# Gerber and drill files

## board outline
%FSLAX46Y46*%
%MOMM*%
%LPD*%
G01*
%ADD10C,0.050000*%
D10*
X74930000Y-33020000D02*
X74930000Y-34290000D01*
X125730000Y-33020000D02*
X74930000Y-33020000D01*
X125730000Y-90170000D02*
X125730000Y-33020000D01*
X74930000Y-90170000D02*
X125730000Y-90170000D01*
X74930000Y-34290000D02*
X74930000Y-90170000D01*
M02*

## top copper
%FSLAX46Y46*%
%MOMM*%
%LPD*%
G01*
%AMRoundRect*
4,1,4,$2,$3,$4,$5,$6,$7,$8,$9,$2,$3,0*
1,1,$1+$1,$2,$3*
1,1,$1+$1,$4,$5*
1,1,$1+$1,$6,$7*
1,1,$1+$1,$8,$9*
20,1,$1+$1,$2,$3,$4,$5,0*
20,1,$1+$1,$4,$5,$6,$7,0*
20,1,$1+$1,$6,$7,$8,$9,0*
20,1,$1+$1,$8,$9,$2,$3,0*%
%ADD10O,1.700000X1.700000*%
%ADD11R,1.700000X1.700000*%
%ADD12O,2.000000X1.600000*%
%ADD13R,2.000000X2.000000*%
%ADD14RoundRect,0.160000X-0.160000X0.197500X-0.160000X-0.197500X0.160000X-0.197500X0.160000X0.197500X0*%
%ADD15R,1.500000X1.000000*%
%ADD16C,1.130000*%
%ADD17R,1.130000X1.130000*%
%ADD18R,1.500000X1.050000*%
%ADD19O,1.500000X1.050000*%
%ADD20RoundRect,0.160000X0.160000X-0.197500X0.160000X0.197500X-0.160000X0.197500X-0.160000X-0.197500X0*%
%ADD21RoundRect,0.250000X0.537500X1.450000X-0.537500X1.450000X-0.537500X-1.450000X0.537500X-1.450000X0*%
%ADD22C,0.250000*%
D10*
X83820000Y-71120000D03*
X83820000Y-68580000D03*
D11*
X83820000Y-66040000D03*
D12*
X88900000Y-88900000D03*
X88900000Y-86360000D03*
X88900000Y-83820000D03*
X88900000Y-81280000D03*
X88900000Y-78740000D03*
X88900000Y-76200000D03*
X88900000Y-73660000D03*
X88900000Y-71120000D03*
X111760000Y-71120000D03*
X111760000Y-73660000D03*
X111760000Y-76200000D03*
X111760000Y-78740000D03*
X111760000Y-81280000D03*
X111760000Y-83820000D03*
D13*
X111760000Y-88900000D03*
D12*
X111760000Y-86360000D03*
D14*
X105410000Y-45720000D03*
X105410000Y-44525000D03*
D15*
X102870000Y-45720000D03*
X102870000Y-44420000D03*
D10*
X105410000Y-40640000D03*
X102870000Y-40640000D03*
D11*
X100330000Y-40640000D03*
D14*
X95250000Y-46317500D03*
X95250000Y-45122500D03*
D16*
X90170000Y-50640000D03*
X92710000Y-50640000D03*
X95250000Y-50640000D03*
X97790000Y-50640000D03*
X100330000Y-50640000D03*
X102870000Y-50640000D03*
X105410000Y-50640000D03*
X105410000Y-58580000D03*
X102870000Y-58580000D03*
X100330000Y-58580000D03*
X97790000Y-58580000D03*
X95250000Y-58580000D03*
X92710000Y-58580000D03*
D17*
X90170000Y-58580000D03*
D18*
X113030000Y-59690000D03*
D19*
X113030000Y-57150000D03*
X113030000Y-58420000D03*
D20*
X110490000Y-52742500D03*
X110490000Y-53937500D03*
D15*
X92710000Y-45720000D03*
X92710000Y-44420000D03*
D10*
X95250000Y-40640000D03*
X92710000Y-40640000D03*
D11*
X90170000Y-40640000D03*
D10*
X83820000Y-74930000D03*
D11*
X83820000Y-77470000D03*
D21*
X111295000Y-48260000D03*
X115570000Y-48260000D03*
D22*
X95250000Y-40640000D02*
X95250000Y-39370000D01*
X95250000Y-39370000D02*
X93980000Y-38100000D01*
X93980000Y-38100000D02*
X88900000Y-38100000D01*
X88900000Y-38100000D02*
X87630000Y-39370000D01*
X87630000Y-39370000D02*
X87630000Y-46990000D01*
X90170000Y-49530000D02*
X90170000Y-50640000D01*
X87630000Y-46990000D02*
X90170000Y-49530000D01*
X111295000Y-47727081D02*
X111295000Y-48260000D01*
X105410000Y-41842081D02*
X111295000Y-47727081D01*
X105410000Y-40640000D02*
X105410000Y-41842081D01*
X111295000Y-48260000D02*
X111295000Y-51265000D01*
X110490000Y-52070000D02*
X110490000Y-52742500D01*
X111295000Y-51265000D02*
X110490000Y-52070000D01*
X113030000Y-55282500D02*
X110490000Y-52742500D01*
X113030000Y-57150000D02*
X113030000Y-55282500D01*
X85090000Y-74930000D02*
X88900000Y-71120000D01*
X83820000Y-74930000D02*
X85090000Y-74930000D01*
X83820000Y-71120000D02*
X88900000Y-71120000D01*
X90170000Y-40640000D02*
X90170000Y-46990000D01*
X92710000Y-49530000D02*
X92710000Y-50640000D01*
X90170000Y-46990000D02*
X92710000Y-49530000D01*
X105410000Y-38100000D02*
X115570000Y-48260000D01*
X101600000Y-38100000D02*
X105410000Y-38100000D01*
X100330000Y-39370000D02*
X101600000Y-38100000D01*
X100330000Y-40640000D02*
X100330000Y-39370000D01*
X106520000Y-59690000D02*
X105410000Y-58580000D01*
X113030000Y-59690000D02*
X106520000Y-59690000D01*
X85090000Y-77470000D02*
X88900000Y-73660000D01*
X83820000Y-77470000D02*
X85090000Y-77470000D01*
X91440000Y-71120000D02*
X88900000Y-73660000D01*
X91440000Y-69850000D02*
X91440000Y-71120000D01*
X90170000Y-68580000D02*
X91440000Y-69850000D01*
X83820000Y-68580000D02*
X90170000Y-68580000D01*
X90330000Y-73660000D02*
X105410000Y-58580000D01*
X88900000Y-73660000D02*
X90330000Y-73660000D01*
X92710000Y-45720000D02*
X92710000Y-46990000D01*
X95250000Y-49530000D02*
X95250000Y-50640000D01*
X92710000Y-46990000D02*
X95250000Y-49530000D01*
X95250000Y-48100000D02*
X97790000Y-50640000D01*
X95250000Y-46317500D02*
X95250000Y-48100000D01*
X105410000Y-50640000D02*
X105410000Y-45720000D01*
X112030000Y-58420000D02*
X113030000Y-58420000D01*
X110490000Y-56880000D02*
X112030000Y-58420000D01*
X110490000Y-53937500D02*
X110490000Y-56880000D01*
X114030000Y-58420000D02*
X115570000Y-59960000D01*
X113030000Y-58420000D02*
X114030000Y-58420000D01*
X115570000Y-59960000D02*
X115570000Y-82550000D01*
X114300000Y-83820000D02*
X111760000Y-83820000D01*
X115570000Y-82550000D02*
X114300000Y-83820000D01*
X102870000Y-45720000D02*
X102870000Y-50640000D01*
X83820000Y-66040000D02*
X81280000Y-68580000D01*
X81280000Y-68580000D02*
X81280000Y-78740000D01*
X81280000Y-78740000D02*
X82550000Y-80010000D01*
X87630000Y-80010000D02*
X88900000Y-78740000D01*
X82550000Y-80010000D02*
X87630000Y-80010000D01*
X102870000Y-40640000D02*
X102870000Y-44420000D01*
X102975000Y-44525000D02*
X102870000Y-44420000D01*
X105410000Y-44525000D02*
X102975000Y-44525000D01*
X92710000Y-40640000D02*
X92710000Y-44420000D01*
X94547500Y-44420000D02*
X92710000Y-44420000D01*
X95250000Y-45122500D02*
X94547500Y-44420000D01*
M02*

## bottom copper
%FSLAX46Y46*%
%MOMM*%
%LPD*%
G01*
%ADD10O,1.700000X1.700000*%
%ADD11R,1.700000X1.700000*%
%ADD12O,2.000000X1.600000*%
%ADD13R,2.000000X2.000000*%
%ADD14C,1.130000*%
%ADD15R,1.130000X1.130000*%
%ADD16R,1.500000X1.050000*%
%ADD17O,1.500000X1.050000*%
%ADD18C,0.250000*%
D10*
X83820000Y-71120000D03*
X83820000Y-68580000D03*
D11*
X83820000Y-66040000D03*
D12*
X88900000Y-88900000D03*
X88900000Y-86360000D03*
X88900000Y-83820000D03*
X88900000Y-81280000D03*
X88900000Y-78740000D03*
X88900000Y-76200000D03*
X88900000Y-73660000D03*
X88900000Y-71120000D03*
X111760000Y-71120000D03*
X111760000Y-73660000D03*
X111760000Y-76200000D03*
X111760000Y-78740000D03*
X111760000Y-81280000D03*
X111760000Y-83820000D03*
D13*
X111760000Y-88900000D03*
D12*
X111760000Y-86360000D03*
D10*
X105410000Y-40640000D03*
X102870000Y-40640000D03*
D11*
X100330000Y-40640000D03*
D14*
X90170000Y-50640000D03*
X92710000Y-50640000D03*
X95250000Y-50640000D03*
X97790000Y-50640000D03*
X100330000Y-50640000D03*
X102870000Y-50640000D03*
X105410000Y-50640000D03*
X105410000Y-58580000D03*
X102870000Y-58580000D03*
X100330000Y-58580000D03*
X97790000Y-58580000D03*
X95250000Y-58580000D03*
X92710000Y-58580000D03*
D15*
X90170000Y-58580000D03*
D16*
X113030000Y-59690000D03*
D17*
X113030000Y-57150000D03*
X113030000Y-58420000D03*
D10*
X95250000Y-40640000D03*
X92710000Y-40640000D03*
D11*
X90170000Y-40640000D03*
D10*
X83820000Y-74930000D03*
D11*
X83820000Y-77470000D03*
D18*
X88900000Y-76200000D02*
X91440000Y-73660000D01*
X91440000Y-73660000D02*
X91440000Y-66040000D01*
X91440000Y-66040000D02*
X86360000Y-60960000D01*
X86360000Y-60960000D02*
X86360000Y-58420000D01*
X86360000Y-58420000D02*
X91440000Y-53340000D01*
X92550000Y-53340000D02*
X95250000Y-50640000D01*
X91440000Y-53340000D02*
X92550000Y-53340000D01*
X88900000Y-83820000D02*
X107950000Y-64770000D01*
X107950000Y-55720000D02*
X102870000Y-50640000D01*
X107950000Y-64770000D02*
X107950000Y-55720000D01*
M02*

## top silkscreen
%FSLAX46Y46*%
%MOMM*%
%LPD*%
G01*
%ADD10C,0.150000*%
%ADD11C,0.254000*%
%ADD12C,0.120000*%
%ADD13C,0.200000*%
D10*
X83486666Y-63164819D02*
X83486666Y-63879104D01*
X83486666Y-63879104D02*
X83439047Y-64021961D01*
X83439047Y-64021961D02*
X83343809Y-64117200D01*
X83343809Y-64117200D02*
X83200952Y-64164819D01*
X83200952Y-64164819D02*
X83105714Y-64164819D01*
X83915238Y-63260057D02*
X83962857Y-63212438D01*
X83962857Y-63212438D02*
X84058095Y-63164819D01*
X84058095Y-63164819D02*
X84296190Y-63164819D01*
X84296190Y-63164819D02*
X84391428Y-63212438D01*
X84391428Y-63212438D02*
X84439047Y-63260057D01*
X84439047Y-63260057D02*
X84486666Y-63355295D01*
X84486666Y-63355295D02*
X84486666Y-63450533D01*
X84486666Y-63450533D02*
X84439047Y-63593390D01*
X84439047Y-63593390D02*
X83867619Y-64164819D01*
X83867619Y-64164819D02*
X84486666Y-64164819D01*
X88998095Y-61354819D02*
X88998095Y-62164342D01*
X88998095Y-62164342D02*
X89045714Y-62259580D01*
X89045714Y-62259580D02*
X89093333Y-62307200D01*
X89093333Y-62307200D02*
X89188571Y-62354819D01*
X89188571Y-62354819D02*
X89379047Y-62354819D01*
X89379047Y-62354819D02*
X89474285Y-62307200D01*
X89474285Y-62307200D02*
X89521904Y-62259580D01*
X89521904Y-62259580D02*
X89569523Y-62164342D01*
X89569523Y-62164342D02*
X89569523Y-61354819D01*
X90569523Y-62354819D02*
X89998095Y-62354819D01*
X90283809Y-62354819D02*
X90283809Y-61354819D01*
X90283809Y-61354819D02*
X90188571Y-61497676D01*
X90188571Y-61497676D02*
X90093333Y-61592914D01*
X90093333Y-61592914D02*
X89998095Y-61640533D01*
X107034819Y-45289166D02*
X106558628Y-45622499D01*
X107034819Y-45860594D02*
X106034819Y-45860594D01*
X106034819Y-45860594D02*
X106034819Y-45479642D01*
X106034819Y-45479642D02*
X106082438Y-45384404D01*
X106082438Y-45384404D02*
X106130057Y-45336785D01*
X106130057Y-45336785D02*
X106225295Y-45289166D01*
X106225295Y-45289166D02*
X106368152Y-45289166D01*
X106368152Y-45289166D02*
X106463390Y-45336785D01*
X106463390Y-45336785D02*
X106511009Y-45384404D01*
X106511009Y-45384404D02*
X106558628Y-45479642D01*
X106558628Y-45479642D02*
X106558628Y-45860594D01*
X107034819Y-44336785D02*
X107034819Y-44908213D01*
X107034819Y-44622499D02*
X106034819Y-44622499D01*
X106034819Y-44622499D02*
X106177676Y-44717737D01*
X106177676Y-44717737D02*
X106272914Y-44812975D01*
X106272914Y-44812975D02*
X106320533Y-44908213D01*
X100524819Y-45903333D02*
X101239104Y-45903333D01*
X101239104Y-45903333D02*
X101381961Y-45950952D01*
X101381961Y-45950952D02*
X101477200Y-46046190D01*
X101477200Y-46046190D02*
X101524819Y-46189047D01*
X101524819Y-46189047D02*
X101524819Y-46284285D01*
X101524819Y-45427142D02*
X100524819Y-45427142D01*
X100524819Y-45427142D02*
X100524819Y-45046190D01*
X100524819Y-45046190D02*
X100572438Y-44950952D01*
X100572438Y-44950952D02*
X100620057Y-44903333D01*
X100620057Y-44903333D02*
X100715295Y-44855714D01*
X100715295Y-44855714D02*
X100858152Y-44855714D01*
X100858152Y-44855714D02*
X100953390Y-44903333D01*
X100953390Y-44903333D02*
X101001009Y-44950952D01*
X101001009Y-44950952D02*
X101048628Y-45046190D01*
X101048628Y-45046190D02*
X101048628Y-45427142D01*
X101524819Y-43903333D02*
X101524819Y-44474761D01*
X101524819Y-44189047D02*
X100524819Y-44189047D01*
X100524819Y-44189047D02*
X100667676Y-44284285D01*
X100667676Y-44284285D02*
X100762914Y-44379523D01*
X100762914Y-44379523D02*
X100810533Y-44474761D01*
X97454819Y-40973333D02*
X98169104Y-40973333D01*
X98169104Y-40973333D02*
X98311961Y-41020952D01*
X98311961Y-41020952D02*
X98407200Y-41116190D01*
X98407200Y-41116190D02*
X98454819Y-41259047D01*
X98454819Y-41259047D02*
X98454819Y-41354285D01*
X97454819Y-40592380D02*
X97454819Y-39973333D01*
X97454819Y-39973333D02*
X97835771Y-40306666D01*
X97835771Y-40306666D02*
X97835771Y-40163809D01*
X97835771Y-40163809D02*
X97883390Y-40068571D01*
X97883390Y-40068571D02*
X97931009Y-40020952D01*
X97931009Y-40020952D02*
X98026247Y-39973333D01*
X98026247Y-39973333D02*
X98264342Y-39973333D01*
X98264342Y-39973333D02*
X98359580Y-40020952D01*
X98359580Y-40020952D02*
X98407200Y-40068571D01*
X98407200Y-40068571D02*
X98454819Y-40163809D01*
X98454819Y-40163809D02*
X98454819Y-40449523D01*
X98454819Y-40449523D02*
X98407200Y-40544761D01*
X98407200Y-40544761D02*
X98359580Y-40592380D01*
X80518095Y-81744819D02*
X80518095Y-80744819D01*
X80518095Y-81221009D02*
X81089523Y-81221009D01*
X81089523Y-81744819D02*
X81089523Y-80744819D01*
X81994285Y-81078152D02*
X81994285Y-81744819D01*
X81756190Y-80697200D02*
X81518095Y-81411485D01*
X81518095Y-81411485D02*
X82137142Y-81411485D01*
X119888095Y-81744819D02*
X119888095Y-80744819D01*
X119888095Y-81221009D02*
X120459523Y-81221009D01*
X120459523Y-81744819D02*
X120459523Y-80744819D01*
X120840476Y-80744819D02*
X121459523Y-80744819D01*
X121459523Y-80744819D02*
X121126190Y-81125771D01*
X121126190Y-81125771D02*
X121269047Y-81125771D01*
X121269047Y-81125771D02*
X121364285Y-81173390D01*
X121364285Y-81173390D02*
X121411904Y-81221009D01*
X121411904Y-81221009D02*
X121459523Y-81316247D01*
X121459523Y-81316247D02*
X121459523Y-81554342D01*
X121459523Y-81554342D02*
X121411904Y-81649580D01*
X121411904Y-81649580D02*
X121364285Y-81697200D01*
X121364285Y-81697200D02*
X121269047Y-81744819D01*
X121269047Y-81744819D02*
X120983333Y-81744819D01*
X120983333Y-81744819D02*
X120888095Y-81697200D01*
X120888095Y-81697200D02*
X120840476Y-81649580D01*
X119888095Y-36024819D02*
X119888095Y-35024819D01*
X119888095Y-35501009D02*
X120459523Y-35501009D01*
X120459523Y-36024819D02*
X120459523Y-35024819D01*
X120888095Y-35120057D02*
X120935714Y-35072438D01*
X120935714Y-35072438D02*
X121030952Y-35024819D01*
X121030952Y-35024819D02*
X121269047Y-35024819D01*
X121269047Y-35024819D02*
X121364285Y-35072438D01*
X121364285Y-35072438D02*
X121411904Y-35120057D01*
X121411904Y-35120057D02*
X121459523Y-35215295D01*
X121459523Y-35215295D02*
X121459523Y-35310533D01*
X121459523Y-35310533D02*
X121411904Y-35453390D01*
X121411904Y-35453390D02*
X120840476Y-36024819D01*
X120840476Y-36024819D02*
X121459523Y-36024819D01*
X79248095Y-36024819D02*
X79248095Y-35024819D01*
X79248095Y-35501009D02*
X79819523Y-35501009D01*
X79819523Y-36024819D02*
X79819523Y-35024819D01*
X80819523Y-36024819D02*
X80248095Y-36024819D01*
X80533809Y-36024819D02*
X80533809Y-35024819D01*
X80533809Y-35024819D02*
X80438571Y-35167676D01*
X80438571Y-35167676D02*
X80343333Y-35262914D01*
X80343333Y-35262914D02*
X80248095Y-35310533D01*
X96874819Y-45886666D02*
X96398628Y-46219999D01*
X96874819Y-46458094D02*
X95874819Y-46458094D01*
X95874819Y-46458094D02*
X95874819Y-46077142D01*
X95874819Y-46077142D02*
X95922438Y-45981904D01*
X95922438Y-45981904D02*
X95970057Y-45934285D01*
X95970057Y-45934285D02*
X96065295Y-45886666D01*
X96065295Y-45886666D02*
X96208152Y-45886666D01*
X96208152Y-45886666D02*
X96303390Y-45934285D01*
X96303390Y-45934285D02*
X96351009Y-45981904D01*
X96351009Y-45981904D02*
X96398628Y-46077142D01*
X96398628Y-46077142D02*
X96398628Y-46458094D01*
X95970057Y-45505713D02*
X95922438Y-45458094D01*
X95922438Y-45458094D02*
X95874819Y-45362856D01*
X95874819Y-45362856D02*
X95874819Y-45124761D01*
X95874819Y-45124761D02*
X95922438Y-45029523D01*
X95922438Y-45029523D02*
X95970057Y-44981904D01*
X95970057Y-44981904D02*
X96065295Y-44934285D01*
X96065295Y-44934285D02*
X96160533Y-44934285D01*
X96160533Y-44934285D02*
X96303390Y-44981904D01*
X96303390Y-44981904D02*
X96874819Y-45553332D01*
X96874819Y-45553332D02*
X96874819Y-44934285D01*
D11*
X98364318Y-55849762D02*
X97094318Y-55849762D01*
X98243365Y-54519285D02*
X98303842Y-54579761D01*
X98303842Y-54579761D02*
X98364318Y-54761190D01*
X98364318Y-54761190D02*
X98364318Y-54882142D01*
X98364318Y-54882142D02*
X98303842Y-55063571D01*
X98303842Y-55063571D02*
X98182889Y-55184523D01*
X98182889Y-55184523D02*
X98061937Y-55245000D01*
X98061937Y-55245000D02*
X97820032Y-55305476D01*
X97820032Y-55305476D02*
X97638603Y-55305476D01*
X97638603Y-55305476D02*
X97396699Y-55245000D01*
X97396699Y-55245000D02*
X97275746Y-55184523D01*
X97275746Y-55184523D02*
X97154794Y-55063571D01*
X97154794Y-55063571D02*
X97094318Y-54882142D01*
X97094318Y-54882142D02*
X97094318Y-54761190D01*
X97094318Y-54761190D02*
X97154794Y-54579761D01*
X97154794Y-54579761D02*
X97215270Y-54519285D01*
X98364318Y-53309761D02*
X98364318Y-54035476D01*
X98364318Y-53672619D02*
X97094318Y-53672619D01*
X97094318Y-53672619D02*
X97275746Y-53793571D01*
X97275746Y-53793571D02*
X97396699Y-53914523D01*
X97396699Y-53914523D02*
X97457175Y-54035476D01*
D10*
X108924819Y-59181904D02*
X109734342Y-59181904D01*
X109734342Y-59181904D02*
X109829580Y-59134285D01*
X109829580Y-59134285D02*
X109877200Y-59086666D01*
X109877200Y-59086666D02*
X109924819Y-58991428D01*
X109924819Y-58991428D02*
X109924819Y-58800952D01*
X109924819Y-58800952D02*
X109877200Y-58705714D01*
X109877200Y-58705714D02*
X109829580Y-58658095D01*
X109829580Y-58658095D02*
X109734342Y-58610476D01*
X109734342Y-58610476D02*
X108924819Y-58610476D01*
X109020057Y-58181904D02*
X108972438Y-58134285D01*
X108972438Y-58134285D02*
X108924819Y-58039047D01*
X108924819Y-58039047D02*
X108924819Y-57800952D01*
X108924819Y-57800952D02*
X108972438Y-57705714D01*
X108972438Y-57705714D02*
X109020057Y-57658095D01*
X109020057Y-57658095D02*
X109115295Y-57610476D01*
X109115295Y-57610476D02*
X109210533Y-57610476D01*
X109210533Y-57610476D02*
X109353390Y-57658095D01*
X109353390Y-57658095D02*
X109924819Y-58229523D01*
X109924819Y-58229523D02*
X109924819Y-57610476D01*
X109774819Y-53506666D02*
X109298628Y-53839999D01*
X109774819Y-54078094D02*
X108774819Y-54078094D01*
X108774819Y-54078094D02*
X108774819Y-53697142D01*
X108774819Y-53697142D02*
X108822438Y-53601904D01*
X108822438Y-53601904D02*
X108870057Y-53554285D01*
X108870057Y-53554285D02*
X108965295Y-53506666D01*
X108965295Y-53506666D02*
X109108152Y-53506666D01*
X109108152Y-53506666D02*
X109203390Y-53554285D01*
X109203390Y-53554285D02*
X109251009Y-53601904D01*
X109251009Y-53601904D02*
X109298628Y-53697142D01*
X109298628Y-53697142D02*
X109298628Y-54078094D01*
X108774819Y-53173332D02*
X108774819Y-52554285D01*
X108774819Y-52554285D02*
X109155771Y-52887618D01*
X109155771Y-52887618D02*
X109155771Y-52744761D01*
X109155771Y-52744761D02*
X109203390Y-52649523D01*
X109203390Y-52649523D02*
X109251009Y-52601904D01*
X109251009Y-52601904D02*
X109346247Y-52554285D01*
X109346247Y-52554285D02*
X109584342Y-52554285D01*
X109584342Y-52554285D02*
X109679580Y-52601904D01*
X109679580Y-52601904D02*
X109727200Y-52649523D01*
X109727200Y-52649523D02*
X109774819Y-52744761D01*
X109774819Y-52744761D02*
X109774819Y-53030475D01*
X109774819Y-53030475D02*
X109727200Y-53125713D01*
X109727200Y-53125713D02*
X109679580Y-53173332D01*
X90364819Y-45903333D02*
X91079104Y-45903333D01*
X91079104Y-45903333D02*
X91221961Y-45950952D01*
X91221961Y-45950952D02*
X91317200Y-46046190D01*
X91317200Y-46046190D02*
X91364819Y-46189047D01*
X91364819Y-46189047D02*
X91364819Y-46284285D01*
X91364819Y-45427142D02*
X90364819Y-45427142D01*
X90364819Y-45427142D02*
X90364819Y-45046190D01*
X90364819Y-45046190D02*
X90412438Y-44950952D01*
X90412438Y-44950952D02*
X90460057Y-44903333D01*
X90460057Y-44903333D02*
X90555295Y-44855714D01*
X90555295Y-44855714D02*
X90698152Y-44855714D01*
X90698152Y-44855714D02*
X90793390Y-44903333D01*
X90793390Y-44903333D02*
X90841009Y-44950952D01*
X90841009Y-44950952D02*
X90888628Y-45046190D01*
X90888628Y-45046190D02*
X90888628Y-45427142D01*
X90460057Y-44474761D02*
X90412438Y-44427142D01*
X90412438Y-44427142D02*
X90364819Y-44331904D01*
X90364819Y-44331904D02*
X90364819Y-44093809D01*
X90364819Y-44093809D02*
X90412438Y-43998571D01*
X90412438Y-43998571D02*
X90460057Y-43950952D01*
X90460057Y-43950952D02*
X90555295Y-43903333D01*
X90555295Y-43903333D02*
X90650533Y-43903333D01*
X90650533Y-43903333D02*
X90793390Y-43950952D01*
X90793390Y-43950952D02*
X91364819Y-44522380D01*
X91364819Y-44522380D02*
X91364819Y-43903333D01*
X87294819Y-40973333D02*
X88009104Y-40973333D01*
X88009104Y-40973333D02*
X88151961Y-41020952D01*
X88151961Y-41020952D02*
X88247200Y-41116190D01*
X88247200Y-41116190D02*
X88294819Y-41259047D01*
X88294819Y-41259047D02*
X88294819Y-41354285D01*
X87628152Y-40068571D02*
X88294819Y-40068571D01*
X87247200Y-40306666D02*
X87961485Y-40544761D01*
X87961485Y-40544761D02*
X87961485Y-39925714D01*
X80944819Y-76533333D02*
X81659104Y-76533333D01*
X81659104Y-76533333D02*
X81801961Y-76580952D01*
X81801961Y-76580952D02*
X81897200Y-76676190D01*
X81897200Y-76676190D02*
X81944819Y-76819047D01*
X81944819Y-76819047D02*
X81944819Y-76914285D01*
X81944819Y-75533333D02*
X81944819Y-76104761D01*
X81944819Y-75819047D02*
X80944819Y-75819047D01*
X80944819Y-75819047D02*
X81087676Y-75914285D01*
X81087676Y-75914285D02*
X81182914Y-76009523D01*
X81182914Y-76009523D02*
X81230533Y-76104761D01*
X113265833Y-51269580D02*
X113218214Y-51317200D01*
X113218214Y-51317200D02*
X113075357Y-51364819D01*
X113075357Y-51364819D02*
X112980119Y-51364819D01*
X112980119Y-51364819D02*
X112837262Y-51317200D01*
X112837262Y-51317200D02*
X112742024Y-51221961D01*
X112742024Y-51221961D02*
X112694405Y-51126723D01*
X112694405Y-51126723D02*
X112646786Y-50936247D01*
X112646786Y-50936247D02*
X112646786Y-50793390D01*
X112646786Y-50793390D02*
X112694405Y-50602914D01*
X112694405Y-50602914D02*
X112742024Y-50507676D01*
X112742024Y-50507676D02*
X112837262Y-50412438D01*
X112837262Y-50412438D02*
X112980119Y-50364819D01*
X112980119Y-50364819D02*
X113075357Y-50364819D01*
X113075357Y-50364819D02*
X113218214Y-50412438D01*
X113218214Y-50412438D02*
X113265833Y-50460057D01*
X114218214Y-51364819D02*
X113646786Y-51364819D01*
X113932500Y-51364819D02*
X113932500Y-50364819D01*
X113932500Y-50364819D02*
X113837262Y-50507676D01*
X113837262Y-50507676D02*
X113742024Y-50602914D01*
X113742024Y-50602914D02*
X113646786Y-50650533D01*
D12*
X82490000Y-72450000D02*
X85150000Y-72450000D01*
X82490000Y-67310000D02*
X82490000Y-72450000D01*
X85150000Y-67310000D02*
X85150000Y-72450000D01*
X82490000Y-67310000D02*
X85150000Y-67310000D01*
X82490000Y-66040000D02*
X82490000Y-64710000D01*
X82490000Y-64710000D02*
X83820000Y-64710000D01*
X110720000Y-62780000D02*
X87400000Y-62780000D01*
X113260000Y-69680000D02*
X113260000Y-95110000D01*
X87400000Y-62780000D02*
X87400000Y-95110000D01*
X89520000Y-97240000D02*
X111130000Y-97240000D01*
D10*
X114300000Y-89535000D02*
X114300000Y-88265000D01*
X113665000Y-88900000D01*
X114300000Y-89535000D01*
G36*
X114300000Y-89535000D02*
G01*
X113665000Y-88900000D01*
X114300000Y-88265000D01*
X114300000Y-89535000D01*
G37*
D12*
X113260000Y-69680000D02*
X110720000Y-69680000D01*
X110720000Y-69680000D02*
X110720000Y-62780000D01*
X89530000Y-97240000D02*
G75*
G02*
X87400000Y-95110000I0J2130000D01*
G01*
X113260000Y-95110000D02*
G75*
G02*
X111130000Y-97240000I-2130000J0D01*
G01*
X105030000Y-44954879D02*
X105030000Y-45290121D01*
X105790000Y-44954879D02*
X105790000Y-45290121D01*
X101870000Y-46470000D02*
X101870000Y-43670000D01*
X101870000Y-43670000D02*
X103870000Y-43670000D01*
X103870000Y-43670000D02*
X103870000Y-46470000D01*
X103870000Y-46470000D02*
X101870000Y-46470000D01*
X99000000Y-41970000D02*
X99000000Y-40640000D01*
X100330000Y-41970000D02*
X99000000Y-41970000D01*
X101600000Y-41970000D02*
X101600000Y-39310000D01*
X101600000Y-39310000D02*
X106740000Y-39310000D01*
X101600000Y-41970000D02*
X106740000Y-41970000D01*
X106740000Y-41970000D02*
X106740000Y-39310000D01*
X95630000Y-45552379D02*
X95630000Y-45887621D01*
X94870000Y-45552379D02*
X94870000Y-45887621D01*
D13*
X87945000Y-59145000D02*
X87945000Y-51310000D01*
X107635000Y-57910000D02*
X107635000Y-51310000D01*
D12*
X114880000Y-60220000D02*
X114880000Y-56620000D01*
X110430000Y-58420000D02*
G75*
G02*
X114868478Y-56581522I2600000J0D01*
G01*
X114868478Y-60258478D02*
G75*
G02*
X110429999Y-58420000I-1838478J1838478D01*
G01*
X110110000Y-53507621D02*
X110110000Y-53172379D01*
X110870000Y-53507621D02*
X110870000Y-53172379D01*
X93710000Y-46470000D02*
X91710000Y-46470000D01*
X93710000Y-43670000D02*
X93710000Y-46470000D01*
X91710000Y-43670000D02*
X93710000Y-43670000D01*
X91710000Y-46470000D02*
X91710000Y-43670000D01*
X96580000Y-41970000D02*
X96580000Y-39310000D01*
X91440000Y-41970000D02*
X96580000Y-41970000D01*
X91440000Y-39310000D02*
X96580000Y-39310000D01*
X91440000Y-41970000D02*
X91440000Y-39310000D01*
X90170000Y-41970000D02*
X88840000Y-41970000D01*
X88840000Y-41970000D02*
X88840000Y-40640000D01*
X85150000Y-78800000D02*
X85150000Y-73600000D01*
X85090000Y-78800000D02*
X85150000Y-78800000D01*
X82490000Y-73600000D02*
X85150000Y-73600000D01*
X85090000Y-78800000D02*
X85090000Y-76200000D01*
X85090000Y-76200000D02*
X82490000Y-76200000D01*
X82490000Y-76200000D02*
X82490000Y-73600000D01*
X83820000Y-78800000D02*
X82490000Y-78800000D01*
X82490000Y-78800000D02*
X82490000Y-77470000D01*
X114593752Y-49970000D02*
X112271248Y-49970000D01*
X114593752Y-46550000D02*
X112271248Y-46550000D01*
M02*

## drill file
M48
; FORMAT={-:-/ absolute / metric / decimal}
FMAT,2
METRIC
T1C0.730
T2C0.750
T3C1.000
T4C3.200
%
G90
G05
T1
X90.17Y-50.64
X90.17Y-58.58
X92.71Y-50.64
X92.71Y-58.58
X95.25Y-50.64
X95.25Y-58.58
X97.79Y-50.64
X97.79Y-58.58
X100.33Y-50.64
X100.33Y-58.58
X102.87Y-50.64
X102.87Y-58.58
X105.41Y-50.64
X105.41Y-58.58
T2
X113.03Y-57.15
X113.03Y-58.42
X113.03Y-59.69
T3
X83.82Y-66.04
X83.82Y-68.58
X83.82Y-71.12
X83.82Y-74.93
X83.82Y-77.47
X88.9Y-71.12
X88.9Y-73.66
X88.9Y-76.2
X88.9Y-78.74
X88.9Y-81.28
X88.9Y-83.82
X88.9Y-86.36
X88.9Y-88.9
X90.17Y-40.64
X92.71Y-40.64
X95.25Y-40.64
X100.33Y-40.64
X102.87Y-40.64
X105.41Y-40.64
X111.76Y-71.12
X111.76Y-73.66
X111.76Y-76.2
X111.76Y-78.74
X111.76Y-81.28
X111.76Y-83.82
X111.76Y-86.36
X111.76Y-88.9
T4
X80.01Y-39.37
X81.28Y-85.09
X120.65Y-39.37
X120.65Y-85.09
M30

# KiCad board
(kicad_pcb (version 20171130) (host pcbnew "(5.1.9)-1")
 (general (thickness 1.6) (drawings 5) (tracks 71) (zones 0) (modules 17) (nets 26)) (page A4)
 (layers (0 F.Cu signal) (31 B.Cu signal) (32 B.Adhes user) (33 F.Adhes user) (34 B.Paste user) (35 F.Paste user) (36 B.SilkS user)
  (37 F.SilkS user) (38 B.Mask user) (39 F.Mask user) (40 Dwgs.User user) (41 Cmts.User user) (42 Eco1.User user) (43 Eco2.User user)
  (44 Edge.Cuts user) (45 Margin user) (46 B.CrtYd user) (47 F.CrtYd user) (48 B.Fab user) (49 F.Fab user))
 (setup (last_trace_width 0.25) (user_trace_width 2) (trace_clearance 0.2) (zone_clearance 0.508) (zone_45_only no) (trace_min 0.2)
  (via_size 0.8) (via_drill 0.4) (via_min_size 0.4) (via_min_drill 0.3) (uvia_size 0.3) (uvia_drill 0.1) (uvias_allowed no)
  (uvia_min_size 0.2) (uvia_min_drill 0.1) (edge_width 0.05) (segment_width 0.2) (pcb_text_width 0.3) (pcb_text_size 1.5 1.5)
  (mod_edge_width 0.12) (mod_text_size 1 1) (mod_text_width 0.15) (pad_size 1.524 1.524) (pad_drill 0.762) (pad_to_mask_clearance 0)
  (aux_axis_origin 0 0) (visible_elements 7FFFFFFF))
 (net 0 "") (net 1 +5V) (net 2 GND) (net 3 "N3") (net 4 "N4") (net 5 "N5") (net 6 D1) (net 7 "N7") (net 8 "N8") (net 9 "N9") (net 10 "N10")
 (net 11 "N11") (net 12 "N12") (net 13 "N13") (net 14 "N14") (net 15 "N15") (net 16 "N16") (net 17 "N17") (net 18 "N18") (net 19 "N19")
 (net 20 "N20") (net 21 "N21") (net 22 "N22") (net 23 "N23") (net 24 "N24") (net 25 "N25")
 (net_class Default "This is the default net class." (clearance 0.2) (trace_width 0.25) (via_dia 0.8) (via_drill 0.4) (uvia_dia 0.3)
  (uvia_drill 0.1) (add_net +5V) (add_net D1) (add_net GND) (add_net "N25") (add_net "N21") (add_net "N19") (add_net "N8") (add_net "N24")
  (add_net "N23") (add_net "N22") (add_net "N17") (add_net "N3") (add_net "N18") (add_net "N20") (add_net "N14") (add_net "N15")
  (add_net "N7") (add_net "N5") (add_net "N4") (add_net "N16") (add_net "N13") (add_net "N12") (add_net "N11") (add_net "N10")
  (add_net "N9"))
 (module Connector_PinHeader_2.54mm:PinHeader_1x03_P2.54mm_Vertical (layer F.Cu) (at 83.82 66.04)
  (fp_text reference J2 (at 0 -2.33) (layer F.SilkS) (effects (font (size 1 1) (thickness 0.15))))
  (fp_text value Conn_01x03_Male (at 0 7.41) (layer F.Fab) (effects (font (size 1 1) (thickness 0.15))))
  (fp_line (start -1.33 6.41) (end 1.33 6.41) (layer F.SilkS) (width 0.12))
  (fp_line (start -1.33 1.27) (end -1.33 6.41) (layer F.SilkS) (width 0.12))
  (fp_line (start 1.33 1.27) (end 1.33 6.41) (layer F.SilkS) (width 0.12))
  (fp_line (start -1.33 1.27) (end 1.33 1.27) (layer F.SilkS) (width 0.12))
  (fp_line (start -1.33 0) (end -1.33 -1.33) (layer F.SilkS) (width 0.12))
  (fp_line (start -1.33 -1.33) (end 0 -1.33) (layer F.SilkS) (width 0.12))
  (pad 3 thru_hole oval (at 0 5.08) (size 1.7 1.7) (drill 1) (layers *.Cu *.Mask) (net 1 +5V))
  (pad 2 thru_hole oval (at 0 2.54) (size 1.7 1.7) (drill 1) (layers *.Cu *.Mask) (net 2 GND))
  (pad 1 thru_hole rect (at 0 0) (size 1.7 1.7) (drill 1) (layers *.Cu *.Mask) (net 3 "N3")))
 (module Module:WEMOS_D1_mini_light (layer F.Cu) (at 111.76 88.9 180)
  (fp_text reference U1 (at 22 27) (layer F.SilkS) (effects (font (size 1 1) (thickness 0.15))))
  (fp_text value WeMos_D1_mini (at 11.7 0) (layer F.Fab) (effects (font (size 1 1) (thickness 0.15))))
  (fp_line (start 1.04 26.12) (end 24.36 26.12) (layer F.SilkS) (width 0.12))
  (fp_line (start -1.5 19.22) (end -1.5 -6.21) (layer F.SilkS) (width 0.12))
  (fp_line (start 24.36 26.12) (end 24.36 -6.21) (layer F.SilkS) (width 0.12))
  (fp_line (start 22.24 -8.34) (end 0.63 -8.34) (layer F.SilkS) (width 0.12))
  (fp_poly (pts (xy -2.54 -0.635) (xy -2.54 0.635) (xy -1.905 0)) (layer F.SilkS) (width 0.15))
  (fp_line (start -1.5 19.22) (end 1.04 19.22) (layer F.SilkS) (width 0.12))
  (fp_line (start 1.04 19.22) (end 1.04 26.12) (layer F.SilkS) (width 0.12))
  (fp_arc (start 22.23 -6.21) (end 24.36 -6.21) (angle -90) (layer F.SilkS) (width 0.12))
  (fp_arc (start 0.63 -6.21) (end 0.63 -8.34) (angle -90) (layer F.SilkS) (width 0.12))
  (pad 16 thru_hole oval (at 22.86 0 180) (size 2 1.6) (drill 1) (layers *.Cu *.Mask) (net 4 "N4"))
  (pad 15 thru_hole oval (at 22.86 2.54 180) (size 2 1.6) (drill 1) (layers *.Cu *.Mask) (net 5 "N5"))
  (pad 14 thru_hole oval (at 22.86 5.08 180) (size 2 1.6) (drill 1) (layers *.Cu *.Mask) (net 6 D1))
  (pad 13 thru_hole oval (at 22.86 7.62 180) (size 2 1.6) (drill 1) (layers *.Cu *.Mask) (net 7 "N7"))
  (pad 12 thru_hole oval (at 22.86 10.16 180) (size 2 1.6) (drill 1) (layers *.Cu *.Mask) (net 3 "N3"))
  (pad 11 thru_hole oval (at 22.86 12.7 180) (size 2 1.6) (drill 1) (layers *.Cu *.Mask) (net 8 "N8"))
  (pad 10 thru_hole oval (at 22.86 15.24 180) (size 2 1.6) (drill 1) (layers *.Cu *.Mask) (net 2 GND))
  (pad 9 thru_hole oval (at 22.86 17.78 180) (size 2 1.6) (drill 1) (layers *.Cu *.Mask) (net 1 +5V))
  (pad 8 thru_hole oval (at 0 17.78 180) (size 2 1.6) (drill 1) (layers *.Cu *.Mask) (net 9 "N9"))
  (pad 7 thru_hole oval (at 0 15.24 180) (size 2 1.6) (drill 1) (layers *.Cu *.Mask) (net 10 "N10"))
  (pad 6 thru_hole oval (at 0 12.7 180) (size 2 1.6) (drill 1) (layers *.Cu *.Mask) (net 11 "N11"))
  (pad 5 thru_hole oval (at 0 10.16 180) (size 2 1.6) (drill 1) (layers *.Cu *.Mask) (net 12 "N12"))
  (pad 4 thru_hole oval (at 0 7.62 180) (size 2 1.6) (drill 1) (layers *.Cu *.Mask) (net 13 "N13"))
  (pad 3 thru_hole oval (at 0 5.08 180) (size 2 1.6) (drill 1) (layers *.Cu *.Mask) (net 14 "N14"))
  (pad 1 thru_hole rect (at 0 0 180) (size 2 2) (drill 1) (layers *.Cu *.Mask) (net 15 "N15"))
  (pad 2 thru_hole oval (at 0 2.54 180) (size 2 1.6) (drill 1) (layers *.Cu *.Mask) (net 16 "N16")))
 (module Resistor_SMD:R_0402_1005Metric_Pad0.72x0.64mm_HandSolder (layer F.Cu) (at 105.41 45.1225 270)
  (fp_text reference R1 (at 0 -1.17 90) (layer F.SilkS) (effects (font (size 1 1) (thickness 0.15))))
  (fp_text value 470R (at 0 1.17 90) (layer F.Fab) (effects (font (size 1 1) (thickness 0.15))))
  (fp_line (start -0.167621 0.38) (end 0.167621 0.38) (layer F.SilkS) (width 0.12))
  (fp_line (start -0.167621 -0.38) (end 0.167621 -0.38) (layer F.SilkS) (width 0.12))
  (pad 2 smd roundrect (at 0.5975 0 270) (size 0.715 0.64) (layers F.Cu F.Paste F.Mask) (roundrect_rratio 0.25) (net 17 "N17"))
  (pad 1 smd roundrect (at -0.5975 0 270) (size 0.715 0.64) (layers F.Cu F.Paste F.Mask) (roundrect_rratio 0.25) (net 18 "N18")))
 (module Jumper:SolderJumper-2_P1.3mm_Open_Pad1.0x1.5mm (layer F.Cu) (at 102.87 45.07 90)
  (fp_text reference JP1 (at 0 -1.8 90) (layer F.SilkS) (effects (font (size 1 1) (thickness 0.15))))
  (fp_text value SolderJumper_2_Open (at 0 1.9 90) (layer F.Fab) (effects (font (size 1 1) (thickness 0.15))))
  (fp_line (start -1.4 -1) (end 1.4 -1) (layer F.SilkS) (width 0.12))
  (fp_line (start 1.4 -1) (end 1.4 1) (layer F.SilkS) (width 0.12))
  (fp_line (start 1.4 1) (end -1.4 1) (layer F.SilkS) (width 0.12))
  (fp_line (start -1.4 1) (end -1.4 -1) (layer F.SilkS) (width 0.12))
  (pad 1 smd rect (at -0.65 0 90) (size 1 1.5) (layers F.Cu F.Mask) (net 6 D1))
  (pad 2 smd rect (at 0.65 0 90) (size 1 1.5) (layers F.Cu F.Mask) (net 18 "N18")))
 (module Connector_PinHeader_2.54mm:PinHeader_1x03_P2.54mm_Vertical (layer F.Cu) (at 100.33 40.64 90)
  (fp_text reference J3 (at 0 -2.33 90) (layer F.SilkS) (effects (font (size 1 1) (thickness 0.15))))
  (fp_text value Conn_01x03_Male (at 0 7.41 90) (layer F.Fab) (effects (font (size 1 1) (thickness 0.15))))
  (fp_line (start -1.33 -1.33) (end 0 -1.33) (layer F.SilkS) (width 0.12))
  (fp_line (start -1.33 0) (end -1.33 -1.33) (layer F.SilkS) (width 0.12))
  (fp_line (start -1.33 1.27) (end 1.33 1.27) (layer F.SilkS) (width 0.12))
  (fp_line (start 1.33 1.27) (end 1.33 6.41) (layer F.SilkS) (width 0.12))
  (fp_line (start -1.33 1.27) (end -1.33 6.41) (layer F.SilkS) (width 0.12))
  (fp_line (start -1.33 6.41) (end 1.33 6.41) (layer F.SilkS) (width 0.12))
  (pad 3 thru_hole oval (at 0 5.08 90) (size 1.7 1.7) (drill 1) (layers *.Cu *.Mask) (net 1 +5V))
  (pad 2 thru_hole oval (at 0 2.54 90) (size 1.7 1.7) (drill 1) (layers *.Cu *.Mask) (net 18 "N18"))
  (pad 1 thru_hole rect (at 0 0 90) (size 1.7 1.7) (drill 1) (layers *.Cu *.Mask) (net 2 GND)))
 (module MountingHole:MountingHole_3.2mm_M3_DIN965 (layer F.Cu) (at 81.28 85.09)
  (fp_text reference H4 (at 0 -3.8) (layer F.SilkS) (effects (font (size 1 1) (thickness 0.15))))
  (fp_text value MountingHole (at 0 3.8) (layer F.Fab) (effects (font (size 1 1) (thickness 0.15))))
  (pad 1 np_thru_hole circle (at 0 0) (size 3.2 3.2) (drill 3.2) (layers *.Cu *.Mask)))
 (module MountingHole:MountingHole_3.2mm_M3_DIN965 (layer F.Cu) (at 120.65 85.09)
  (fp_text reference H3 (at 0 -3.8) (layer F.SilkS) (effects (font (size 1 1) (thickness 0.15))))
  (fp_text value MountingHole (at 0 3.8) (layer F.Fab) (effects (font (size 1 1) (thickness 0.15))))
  (pad 1 np_thru_hole circle (at 0 0) (size 3.2 3.2) (drill 3.2) (layers *.Cu *.Mask)))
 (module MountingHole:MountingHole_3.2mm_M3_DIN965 (layer F.Cu) (at 120.65 39.37)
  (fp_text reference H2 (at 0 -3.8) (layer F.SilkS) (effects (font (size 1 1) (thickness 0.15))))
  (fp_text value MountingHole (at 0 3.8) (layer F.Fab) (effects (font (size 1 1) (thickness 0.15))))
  (pad 1 np_thru_hole circle (at 0 0) (size 3.2 3.2) (drill 3.2) (layers *.Cu *.Mask)))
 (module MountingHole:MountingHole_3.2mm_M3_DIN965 (layer F.Cu) (at 80.01 39.37)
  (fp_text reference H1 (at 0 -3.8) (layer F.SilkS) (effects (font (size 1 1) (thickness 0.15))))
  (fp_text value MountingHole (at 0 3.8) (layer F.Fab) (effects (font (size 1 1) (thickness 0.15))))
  (pad 1 np_thru_hole circle (at 0 0) (size 3.2 3.2) (drill 3.2) (layers *.Cu *.Mask)))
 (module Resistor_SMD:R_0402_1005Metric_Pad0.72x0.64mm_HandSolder (layer F.Cu) (at 95.25 45.72 270)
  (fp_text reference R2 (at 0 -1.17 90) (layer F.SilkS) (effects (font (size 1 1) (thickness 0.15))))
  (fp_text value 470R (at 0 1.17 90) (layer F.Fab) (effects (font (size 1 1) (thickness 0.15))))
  (fp_line (start -0.167621 -0.38) (end 0.167621 -0.38) (layer F.SilkS) (width 0.12))
  (fp_line (start -0.167621 0.38) (end 0.167621 0.38) (layer F.SilkS) (width 0.12))
  (pad 2 smd roundrect (at 0.5975 0 270) (size 0.715 0.64) (layers F.Cu F.Paste F.Mask) (roundrect_rratio 0.25) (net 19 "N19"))
  (pad 1 smd roundrect (at -0.5975 0 270) (size 0.715 0.64) (layers F.Cu F.Paste F.Mask) (roundrect_rratio 0.25) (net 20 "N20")))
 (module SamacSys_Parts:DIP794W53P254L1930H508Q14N (layer F.Cu) (at 97.79 54.61 90)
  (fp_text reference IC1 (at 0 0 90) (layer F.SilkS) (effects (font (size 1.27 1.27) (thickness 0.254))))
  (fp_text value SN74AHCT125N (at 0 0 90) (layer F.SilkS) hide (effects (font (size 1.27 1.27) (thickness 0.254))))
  (fp_line (start -4.535 -9.845) (end 3.3 -9.845) (layer F.SilkS) (width 0.2))
  (fp_line (start -3.3 9.845) (end 3.3 9.845) (layer F.SilkS) (width 0.2))
  (pad 14 thru_hole circle (at 3.97 -7.62 90) (size 1.13 1.13) (drill 0.73) (layers *.Cu *.Mask) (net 1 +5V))
  (pad 13 thru_hole circle (at 3.97 -5.08 90) (size 1.13 1.13) (drill 0.73) (layers *.Cu *.Mask) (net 2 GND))
  (pad 12 thru_hole circle (at 3.97 -2.54 90) (size 1.13 1.13) (drill 0.73) (layers *.Cu *.Mask) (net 8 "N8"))
  (pad 11 thru_hole circle (at 3.97 0 90) (size 1.13 1.13) (drill 0.73) (layers *.Cu *.Mask) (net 19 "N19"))
  (pad 10 thru_hole circle (at 3.97 2.54 90) (size 1.13 1.13) (drill 0.73) (layers *.Cu *.Mask) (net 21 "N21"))
  (pad 9 thru_hole circle (at 3.97 5.08 90) (size 1.13 1.13) (drill 0.73) (layers *.Cu *.Mask) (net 6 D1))
  (pad 8 thru_hole circle (at 3.97 7.62 90) (size 1.13 1.13) (drill 0.73) (layers *.Cu *.Mask) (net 17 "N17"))
  (pad 7 thru_hole circle (at -3.97 7.62 90) (size 1.13 1.13) (drill 0.73) (layers *.Cu *.Mask) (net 2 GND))
  (pad 6 thru_hole circle (at -3.97 5.08 90) (size 1.13 1.13) (drill 0.73) (layers *.Cu *.Mask) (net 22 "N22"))
  (pad 5 thru_hole circle (at -3.97 2.54 90) (size 1.13 1.13) (drill 0.73) (layers *.Cu *.Mask) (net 1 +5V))
  (pad 4 thru_hole circle (at -3.97 0 90) (size 1.13 1.13) (drill 0.73) (layers *.Cu *.Mask) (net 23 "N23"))
  (pad 3 thru_hole circle (at -3.97 -2.54 90) (size 1.13 1.13) (drill 0.73) (layers *.Cu *.Mask) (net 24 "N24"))
  (pad 2 thru_hole circle (at -3.97 -5.08 90) (size 1.13 1.13) (drill 0.73) (layers *.Cu *.Mask) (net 1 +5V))
  (pad 1 thru_hole rect (at -3.97 -7.62 90) (size 1.13 1.13) (drill 0.73) (layers *.Cu *.Mask) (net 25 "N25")))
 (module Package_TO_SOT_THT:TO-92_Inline (layer F.Cu) (at 113.03 59.69 90)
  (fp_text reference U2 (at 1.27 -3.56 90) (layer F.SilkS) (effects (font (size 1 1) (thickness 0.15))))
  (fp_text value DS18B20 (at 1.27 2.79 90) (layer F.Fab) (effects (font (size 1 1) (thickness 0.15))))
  (fp_line (start -0.53 1.85) (end 3.07 1.85) (layer F.SilkS) (width 0.12))
  (fp_arc (start 1.27 0) (end 1.27 -2.6) (angle 135) (layer F.SilkS) (width 0.12))
  (fp_arc (start 1.27 0) (end 1.27 -2.6) (angle -135) (layer F.SilkS) (width 0.12))
  (pad 1 thru_hole rect (at 0 0 90) (size 1.05 1.5) (drill 0.75) (layers *.Cu *.Mask) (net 2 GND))
  (pad 3 thru_hole oval (at 2.54 0 90) (size 1.05 1.5) (drill 0.75) (layers *.Cu *.Mask) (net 1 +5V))
  (pad 2 thru_hole oval (at 1.27 0 90) (size 1.05 1.5) (drill 0.75) (layers *.Cu *.Mask) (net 14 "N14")))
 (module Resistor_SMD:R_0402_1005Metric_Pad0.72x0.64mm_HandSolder (layer F.Cu) (at 110.49 53.34 90)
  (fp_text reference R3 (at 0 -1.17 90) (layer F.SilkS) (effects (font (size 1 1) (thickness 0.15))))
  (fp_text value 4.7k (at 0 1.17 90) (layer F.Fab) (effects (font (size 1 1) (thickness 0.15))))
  (fp_line (start -0.167621 -0.38) (end 0.167621 -0.38) (layer F.SilkS) (width 0.12))
  (fp_line (start -0.167621 0.38) (end 0.167621 0.38) (layer F.SilkS) (width 0.12))
  (pad 2 smd roundrect (at 0.5975 0 90) (size 0.715 0.64) (layers F.Cu F.Paste F.Mask) (roundrect_rratio 0.25) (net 1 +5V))
  (pad 1 smd roundrect (at -0.5975 0 90) (size 0.715 0.64) (layers F.Cu F.Paste F.Mask) (roundrect_rratio 0.25) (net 14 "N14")))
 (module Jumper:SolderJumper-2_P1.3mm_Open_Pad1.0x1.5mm (layer F.Cu) (at 92.71 45.07 90)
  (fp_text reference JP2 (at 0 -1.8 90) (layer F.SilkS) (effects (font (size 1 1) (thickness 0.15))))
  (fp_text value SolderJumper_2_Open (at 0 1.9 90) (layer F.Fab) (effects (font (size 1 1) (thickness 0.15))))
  (fp_line (start -1.4 1) (end -1.4 -1) (layer F.SilkS) (width 0.12))
  (fp_line (start 1.4 1) (end -1.4 1) (layer F.SilkS) (width 0.12))
  (fp_line (start 1.4 -1) (end 1.4 1) (layer F.SilkS) (width 0.12))
  (fp_line (start -1.4 -1) (end 1.4 -1) (layer F.SilkS) (width 0.12))
  (pad 1 smd rect (at -0.65 0 90) (size 1 1.5) (layers F.Cu F.Mask) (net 8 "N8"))
  (pad 2 smd rect (at 0.65 0 90) (size 1 1.5) (layers F.Cu F.Mask) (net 20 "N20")))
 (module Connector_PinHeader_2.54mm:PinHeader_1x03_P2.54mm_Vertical (layer F.Cu) (at 90.17 40.64 90)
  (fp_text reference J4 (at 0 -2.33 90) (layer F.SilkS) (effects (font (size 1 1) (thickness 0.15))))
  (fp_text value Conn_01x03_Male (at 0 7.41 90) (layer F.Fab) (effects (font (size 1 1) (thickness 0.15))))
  (fp_line (start -1.33 6.41) (end 1.33 6.41) (layer F.SilkS) (width 0.12))
  (fp_line (start -1.33 1.27) (end -1.33 6.41) (layer F.SilkS) (width 0.12))
  (fp_line (start 1.33 1.27) (end 1.33 6.41) (layer F.SilkS) (width 0.12))
  (fp_line (start -1.33 1.27) (end 1.33 1.27) (layer F.SilkS) (width 0.12))
  (fp_line (start -1.33 0) (end -1.33 -1.33) (layer F.SilkS) (width 0.12))
  (fp_line (start -1.33 -1.33) (end 0 -1.33) (layer F.SilkS) (width 0.12))
  (pad 3 thru_hole oval (at 0 5.08 90) (size 1.7 1.7) (drill 1) (layers *.Cu *.Mask) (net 1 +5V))
  (pad 2 thru_hole oval (at 0 2.54 90) (size 1.7 1.7) (drill 1) (layers *.Cu *.Mask) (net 20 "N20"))
  (pad 1 thru_hole rect (at 0 0 90) (size 1.7 1.7) (drill 1) (layers *.Cu *.Mask) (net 2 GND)))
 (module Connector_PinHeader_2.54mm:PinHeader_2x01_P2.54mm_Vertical (layer F.Cu) (at 83.82 77.47 90)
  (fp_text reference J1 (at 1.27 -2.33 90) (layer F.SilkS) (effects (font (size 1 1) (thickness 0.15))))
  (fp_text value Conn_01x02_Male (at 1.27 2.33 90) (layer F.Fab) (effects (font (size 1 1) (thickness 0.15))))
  (fp_line (start -1.33 1.33) (end 3.87 1.33) (layer F.SilkS) (width 0.12))
  (fp_line (start -1.33 1.27) (end -1.33 1.33) (layer F.SilkS) (width 0.12))
  (fp_line (start 3.87 -1.33) (end 3.87 1.33) (layer F.SilkS) (width 0.12))
  (fp_line (start -1.33 1.27) (end 1.27 1.27) (layer F.SilkS) (width 0.12))
  (fp_line (start 1.27 1.27) (end 1.27 -1.33) (layer F.SilkS) (width 0.12))
  (fp_line (start 1.27 -1.33) (end 3.87 -1.33) (layer F.SilkS) (width 0.12))
  (fp_line (start -1.33 0) (end -1.33 -1.33) (layer F.SilkS) (width 0.12))
  (fp_line (start -1.33 -1.33) (end 0 -1.33) (layer F.SilkS) (width 0.12))
  (pad 2 thru_hole oval (at 2.54 0 90) (size 1.7 1.7) (drill 1) (layers *.Cu *.Mask) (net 1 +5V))
  (pad 1 thru_hole rect (at 0 0 90) (size 1.7 1.7) (drill 1) (layers *.Cu *.Mask) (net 2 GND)))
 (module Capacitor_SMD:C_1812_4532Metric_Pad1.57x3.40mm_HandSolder (layer F.Cu) (at 113.4325 48.26 180)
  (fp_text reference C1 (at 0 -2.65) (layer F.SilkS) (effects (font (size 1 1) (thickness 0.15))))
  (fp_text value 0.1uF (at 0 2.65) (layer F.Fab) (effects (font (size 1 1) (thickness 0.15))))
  (fp_line (start -1.161252 -1.71) (end 1.161252 -1.71) (layer F.SilkS) (width 0.12))
  (fp_line (start -1.161252 1.71) (end 1.161252 1.71) (layer F.SilkS) (width 0.12))
  (pad 2 smd roundrect (at 2.1375 0 180) (size 1.575 3.4) (layers F.Cu F.Paste F.Mask) (roundrect_rratio 0.15873) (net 1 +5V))
  (pad 1 smd roundrect (at -2.1375 0 180) (size 1.575 3.4) (layers F.Cu F.Paste F.Mask) (roundrect_rratio 0.15873) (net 2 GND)))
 (gr_line (start 74.93 33.02) (end 74.93 34.29) (layer Edge.Cuts) (width 0.05))
 (gr_line (start 125.73 33.02) (end 74.93 33.02) (layer Edge.Cuts) (width 0.05))
 (gr_line (start 125.73 90.17) (end 125.73 33.02) (layer Edge.Cuts) (width 0.05))
 (gr_line (start 74.93 90.17) (end 125.73 90.17) (layer Edge.Cuts) (width 0.05))
 (gr_line (start 74.93 34.29) (end 74.93 90.17) (layer Edge.Cuts) (width 0.05))
 (segment (start 95.25 40.64) (end 95.25 39.37) (width 0.25) (layer F.Cu) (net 1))
 (segment (start 95.25 39.37) (end 93.98 38.1) (width 0.25) (layer F.Cu) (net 1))
 (segment (start 93.98 38.1) (end 88.9 38.1) (width 0.25) (layer F.Cu) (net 1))
 (segment (start 88.9 38.1) (end 87.63 39.37) (width 0.25) (layer F.Cu) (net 1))
 (segment (start 87.63 39.37) (end 87.63 46.99) (width 0.25) (layer F.Cu) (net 1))
 (segment (start 90.17 49.53) (end 90.17 50.64) (width 0.25) (layer F.Cu) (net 1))
 (segment (start 87.63 46.99) (end 90.17 49.53) (width 0.25) (layer F.Cu) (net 1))
 (segment (start 111.295 47.727081) (end 111.295 48.26) (width 0.25) (layer F.Cu) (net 1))
 (segment (start 105.41 41.842081) (end 111.295 47.727081) (width 0.25) (layer F.Cu) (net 1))
 (segment (start 105.41 40.64) (end 105.41 41.842081) (width 0.25) (layer F.Cu) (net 1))
 (segment (start 111.295 48.26) (end 111.295 51.265) (width 0.25) (layer F.Cu) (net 1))
 (segment (start 110.49 52.07) (end 110.49 52.7425) (width 0.25) (layer F.Cu) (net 1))
 (segment (start 111.295 51.265) (end 110.49 52.07) (width 0.25) (layer F.Cu) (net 1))
 (segment (start 113.03 55.2825) (end 110.49 52.7425) (width 0.25) (layer F.Cu) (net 1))
 (segment (start 113.03 57.15) (end 113.03 55.2825) (width 0.25) (layer F.Cu) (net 1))
 (segment (start 85.09 74.93) (end 88.9 71.12) (width 0.25) (layer F.Cu) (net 1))
 (segment (start 83.82 74.93) (end 85.09 74.93) (width 0.25) (layer F.Cu) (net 1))
 (segment (start 83.82 71.12) (end 88.9 71.12) (width 0.25) (layer F.Cu) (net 1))
 (segment (start 90.17 40.64) (end 90.17 46.99) (width 0.25) (layer F.Cu) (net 2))
 (segment (start 92.71 49.53) (end 92.71 50.64) (width 0.25) (layer F.Cu) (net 2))
 (segment (start 90.17 46.99) (end 92.71 49.53) (width 0.25) (layer F.Cu) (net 2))
 (segment (start 105.41 38.1) (end 115.57 48.26) (width 0.25) (layer F.Cu) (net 2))
 (segment (start 101.6 38.1) (end 105.41 38.1) (width 0.25) (layer F.Cu) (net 2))
 (segment (start 100.33 39.37) (end 101.6 38.1) (width 0.25) (layer F.Cu) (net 2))
 (segment (start 100.33 40.64) (end 100.33 39.37) (width 0.25) (layer F.Cu) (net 2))
 (segment (start 106.52 59.69) (end 105.41 58.58) (width 0.25) (layer F.Cu) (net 2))
 (segment (start 113.03 59.69) (end 106.52 59.69) (width 0.25) (layer F.Cu) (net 2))
 (segment (start 85.09 77.47) (end 88.9 73.66) (width 0.25) (layer F.Cu) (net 2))
 (segment (start 83.82 77.47) (end 85.09 77.47) (width 0.25) (layer F.Cu) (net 2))
 (segment (start 91.44 71.12) (end 88.9 73.66) (width 0.25) (layer F.Cu) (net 2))
 (segment (start 91.44 69.85) (end 91.44 71.12) (width 0.25) (layer F.Cu) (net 2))
 (segment (start 90.17 68.58) (end 91.44 69.85) (width 0.25) (layer F.Cu) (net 2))
 (segment (start 83.82 68.58) (end 90.17 68.58) (width 0.25) (layer F.Cu) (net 2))
 (segment (start 90.33 73.66) (end 105.41 58.58) (width 0.25) (layer F.Cu) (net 2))
 (segment (start 88.9 73.66) (end 90.33 73.66) (width 0.25) (layer F.Cu) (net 2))
 (segment (start 92.71 45.72) (end 92.71 46.99) (width 0.25) (layer F.Cu) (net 8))
 (segment (start 95.25 49.53) (end 95.25 50.64) (width 0.25) (layer F.Cu) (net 8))
 (segment (start 92.71 46.99) (end 95.25 49.53) (width 0.25) (layer F.Cu) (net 8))
 (segment (start 88.9 76.2) (end 91.44 73.66) (width 0.25) (layer B.Cu) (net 8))
 (segment (start 91.44 73.66) (end 91.44 66.04) (width 0.25) (layer B.Cu) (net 8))
 (segment (start 91.44 66.04) (end 86.36 60.96) (width 0.25) (layer B.Cu) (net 8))
 (segment (start 86.36 60.96) (end 86.36 58.42) (width 0.25) (layer B.Cu) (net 8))
 (segment (start 86.36 58.42) (end 91.44 53.34) (width 0.25) (layer B.Cu) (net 8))
 (segment (start 92.55 53.34) (end 95.25 50.64) (width 0.25) (layer B.Cu) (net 8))
 (segment (start 91.44 53.34) (end 92.55 53.34) (width 0.25) (layer B.Cu) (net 8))
 (segment (start 95.25 48.1) (end 97.79 50.64) (width 0.25) (layer F.Cu) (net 19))
 (segment (start 95.25 46.3175) (end 95.25 48.1) (width 0.25) (layer F.Cu) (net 19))
 (segment (start 105.41 50.64) (end 105.41 45.72) (width 0.25) (layer F.Cu) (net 17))
 (segment (start 112.03 58.42) (end 113.03 58.42) (width 0.25) (layer F.Cu) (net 14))
 (segment (start 110.49 56.88) (end 112.03 58.42) (width 0.25) (layer F.Cu) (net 14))
 (segment (start 110.49 53.9375) (end 110.49 56.88) (width 0.25) (layer F.Cu) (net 14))
 (segment (start 114.03 58.42) (end 115.57 59.96) (width 0.25) (layer F.Cu) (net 14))
 (segment (start 113.03 58.42) (end 114.03 58.42) (width 0.25) (layer F.Cu) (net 14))
 (segment (start 115.57 59.96) (end 115.57 82.55) (width 0.25) (layer F.Cu) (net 14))
 (segment (start 114.3 83.82) (end 111.76 83.82) (width 0.25) (layer F.Cu) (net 14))
 (segment (start 115.57 82.55) (end 114.3 83.82) (width 0.25) (layer F.Cu) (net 14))
 (segment (start 102.87 45.72) (end 102.87 50.64) (width 0.25) (layer F.Cu) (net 6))
 (segment (start 88.9 83.82) (end 107.95 64.77) (width 0.25) (layer B.Cu) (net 6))
 (segment (start 107.95 55.72) (end 102.87 50.64) (width 0.25) (layer B.Cu) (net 6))
 (segment (start 107.95 64.77) (end 107.95 55.72) (width 0.25) (layer B.Cu) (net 6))
 (segment (start 83.82 66.04) (end 81.28 68.58) (width 0.25) (layer F.Cu) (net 3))
 (segment (start 81.28 68.58) (end 81.28 78.74) (width 0.25) (layer F.Cu) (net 3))
 (segment (start 81.28 78.74) (end 82.55 80.01) (width 0.25) (layer F.Cu) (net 3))
 (segment (start 87.63 80.01) (end 88.9 78.74) (width 0.25) (layer F.Cu) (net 3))
 (segment (start 82.55 80.01) (end 87.63 80.01) (width 0.25) (layer F.Cu) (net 3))
 (segment (start 102.87 40.64) (end 102.87 44.42) (width 0.25) (layer F.Cu) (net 18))
 (segment (start 102.975 44.525) (end 102.87 44.42) (width 0.25) (layer F.Cu) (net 18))
 (segment (start 105.41 44.525) (end 102.975 44.525) (width 0.25) (layer F.Cu) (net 18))
 (segment (start 92.71 40.64) (end 92.71 44.42) (width 0.25) (layer F.Cu) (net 20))
 (segment (start 94.5475 44.42) (end 92.71 44.42) (width 0.25) (layer F.Cu) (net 20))
 (segment (start 95.25 45.1225) (end 94.5475 44.42) (width 0.25) (layer F.Cu) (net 20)))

